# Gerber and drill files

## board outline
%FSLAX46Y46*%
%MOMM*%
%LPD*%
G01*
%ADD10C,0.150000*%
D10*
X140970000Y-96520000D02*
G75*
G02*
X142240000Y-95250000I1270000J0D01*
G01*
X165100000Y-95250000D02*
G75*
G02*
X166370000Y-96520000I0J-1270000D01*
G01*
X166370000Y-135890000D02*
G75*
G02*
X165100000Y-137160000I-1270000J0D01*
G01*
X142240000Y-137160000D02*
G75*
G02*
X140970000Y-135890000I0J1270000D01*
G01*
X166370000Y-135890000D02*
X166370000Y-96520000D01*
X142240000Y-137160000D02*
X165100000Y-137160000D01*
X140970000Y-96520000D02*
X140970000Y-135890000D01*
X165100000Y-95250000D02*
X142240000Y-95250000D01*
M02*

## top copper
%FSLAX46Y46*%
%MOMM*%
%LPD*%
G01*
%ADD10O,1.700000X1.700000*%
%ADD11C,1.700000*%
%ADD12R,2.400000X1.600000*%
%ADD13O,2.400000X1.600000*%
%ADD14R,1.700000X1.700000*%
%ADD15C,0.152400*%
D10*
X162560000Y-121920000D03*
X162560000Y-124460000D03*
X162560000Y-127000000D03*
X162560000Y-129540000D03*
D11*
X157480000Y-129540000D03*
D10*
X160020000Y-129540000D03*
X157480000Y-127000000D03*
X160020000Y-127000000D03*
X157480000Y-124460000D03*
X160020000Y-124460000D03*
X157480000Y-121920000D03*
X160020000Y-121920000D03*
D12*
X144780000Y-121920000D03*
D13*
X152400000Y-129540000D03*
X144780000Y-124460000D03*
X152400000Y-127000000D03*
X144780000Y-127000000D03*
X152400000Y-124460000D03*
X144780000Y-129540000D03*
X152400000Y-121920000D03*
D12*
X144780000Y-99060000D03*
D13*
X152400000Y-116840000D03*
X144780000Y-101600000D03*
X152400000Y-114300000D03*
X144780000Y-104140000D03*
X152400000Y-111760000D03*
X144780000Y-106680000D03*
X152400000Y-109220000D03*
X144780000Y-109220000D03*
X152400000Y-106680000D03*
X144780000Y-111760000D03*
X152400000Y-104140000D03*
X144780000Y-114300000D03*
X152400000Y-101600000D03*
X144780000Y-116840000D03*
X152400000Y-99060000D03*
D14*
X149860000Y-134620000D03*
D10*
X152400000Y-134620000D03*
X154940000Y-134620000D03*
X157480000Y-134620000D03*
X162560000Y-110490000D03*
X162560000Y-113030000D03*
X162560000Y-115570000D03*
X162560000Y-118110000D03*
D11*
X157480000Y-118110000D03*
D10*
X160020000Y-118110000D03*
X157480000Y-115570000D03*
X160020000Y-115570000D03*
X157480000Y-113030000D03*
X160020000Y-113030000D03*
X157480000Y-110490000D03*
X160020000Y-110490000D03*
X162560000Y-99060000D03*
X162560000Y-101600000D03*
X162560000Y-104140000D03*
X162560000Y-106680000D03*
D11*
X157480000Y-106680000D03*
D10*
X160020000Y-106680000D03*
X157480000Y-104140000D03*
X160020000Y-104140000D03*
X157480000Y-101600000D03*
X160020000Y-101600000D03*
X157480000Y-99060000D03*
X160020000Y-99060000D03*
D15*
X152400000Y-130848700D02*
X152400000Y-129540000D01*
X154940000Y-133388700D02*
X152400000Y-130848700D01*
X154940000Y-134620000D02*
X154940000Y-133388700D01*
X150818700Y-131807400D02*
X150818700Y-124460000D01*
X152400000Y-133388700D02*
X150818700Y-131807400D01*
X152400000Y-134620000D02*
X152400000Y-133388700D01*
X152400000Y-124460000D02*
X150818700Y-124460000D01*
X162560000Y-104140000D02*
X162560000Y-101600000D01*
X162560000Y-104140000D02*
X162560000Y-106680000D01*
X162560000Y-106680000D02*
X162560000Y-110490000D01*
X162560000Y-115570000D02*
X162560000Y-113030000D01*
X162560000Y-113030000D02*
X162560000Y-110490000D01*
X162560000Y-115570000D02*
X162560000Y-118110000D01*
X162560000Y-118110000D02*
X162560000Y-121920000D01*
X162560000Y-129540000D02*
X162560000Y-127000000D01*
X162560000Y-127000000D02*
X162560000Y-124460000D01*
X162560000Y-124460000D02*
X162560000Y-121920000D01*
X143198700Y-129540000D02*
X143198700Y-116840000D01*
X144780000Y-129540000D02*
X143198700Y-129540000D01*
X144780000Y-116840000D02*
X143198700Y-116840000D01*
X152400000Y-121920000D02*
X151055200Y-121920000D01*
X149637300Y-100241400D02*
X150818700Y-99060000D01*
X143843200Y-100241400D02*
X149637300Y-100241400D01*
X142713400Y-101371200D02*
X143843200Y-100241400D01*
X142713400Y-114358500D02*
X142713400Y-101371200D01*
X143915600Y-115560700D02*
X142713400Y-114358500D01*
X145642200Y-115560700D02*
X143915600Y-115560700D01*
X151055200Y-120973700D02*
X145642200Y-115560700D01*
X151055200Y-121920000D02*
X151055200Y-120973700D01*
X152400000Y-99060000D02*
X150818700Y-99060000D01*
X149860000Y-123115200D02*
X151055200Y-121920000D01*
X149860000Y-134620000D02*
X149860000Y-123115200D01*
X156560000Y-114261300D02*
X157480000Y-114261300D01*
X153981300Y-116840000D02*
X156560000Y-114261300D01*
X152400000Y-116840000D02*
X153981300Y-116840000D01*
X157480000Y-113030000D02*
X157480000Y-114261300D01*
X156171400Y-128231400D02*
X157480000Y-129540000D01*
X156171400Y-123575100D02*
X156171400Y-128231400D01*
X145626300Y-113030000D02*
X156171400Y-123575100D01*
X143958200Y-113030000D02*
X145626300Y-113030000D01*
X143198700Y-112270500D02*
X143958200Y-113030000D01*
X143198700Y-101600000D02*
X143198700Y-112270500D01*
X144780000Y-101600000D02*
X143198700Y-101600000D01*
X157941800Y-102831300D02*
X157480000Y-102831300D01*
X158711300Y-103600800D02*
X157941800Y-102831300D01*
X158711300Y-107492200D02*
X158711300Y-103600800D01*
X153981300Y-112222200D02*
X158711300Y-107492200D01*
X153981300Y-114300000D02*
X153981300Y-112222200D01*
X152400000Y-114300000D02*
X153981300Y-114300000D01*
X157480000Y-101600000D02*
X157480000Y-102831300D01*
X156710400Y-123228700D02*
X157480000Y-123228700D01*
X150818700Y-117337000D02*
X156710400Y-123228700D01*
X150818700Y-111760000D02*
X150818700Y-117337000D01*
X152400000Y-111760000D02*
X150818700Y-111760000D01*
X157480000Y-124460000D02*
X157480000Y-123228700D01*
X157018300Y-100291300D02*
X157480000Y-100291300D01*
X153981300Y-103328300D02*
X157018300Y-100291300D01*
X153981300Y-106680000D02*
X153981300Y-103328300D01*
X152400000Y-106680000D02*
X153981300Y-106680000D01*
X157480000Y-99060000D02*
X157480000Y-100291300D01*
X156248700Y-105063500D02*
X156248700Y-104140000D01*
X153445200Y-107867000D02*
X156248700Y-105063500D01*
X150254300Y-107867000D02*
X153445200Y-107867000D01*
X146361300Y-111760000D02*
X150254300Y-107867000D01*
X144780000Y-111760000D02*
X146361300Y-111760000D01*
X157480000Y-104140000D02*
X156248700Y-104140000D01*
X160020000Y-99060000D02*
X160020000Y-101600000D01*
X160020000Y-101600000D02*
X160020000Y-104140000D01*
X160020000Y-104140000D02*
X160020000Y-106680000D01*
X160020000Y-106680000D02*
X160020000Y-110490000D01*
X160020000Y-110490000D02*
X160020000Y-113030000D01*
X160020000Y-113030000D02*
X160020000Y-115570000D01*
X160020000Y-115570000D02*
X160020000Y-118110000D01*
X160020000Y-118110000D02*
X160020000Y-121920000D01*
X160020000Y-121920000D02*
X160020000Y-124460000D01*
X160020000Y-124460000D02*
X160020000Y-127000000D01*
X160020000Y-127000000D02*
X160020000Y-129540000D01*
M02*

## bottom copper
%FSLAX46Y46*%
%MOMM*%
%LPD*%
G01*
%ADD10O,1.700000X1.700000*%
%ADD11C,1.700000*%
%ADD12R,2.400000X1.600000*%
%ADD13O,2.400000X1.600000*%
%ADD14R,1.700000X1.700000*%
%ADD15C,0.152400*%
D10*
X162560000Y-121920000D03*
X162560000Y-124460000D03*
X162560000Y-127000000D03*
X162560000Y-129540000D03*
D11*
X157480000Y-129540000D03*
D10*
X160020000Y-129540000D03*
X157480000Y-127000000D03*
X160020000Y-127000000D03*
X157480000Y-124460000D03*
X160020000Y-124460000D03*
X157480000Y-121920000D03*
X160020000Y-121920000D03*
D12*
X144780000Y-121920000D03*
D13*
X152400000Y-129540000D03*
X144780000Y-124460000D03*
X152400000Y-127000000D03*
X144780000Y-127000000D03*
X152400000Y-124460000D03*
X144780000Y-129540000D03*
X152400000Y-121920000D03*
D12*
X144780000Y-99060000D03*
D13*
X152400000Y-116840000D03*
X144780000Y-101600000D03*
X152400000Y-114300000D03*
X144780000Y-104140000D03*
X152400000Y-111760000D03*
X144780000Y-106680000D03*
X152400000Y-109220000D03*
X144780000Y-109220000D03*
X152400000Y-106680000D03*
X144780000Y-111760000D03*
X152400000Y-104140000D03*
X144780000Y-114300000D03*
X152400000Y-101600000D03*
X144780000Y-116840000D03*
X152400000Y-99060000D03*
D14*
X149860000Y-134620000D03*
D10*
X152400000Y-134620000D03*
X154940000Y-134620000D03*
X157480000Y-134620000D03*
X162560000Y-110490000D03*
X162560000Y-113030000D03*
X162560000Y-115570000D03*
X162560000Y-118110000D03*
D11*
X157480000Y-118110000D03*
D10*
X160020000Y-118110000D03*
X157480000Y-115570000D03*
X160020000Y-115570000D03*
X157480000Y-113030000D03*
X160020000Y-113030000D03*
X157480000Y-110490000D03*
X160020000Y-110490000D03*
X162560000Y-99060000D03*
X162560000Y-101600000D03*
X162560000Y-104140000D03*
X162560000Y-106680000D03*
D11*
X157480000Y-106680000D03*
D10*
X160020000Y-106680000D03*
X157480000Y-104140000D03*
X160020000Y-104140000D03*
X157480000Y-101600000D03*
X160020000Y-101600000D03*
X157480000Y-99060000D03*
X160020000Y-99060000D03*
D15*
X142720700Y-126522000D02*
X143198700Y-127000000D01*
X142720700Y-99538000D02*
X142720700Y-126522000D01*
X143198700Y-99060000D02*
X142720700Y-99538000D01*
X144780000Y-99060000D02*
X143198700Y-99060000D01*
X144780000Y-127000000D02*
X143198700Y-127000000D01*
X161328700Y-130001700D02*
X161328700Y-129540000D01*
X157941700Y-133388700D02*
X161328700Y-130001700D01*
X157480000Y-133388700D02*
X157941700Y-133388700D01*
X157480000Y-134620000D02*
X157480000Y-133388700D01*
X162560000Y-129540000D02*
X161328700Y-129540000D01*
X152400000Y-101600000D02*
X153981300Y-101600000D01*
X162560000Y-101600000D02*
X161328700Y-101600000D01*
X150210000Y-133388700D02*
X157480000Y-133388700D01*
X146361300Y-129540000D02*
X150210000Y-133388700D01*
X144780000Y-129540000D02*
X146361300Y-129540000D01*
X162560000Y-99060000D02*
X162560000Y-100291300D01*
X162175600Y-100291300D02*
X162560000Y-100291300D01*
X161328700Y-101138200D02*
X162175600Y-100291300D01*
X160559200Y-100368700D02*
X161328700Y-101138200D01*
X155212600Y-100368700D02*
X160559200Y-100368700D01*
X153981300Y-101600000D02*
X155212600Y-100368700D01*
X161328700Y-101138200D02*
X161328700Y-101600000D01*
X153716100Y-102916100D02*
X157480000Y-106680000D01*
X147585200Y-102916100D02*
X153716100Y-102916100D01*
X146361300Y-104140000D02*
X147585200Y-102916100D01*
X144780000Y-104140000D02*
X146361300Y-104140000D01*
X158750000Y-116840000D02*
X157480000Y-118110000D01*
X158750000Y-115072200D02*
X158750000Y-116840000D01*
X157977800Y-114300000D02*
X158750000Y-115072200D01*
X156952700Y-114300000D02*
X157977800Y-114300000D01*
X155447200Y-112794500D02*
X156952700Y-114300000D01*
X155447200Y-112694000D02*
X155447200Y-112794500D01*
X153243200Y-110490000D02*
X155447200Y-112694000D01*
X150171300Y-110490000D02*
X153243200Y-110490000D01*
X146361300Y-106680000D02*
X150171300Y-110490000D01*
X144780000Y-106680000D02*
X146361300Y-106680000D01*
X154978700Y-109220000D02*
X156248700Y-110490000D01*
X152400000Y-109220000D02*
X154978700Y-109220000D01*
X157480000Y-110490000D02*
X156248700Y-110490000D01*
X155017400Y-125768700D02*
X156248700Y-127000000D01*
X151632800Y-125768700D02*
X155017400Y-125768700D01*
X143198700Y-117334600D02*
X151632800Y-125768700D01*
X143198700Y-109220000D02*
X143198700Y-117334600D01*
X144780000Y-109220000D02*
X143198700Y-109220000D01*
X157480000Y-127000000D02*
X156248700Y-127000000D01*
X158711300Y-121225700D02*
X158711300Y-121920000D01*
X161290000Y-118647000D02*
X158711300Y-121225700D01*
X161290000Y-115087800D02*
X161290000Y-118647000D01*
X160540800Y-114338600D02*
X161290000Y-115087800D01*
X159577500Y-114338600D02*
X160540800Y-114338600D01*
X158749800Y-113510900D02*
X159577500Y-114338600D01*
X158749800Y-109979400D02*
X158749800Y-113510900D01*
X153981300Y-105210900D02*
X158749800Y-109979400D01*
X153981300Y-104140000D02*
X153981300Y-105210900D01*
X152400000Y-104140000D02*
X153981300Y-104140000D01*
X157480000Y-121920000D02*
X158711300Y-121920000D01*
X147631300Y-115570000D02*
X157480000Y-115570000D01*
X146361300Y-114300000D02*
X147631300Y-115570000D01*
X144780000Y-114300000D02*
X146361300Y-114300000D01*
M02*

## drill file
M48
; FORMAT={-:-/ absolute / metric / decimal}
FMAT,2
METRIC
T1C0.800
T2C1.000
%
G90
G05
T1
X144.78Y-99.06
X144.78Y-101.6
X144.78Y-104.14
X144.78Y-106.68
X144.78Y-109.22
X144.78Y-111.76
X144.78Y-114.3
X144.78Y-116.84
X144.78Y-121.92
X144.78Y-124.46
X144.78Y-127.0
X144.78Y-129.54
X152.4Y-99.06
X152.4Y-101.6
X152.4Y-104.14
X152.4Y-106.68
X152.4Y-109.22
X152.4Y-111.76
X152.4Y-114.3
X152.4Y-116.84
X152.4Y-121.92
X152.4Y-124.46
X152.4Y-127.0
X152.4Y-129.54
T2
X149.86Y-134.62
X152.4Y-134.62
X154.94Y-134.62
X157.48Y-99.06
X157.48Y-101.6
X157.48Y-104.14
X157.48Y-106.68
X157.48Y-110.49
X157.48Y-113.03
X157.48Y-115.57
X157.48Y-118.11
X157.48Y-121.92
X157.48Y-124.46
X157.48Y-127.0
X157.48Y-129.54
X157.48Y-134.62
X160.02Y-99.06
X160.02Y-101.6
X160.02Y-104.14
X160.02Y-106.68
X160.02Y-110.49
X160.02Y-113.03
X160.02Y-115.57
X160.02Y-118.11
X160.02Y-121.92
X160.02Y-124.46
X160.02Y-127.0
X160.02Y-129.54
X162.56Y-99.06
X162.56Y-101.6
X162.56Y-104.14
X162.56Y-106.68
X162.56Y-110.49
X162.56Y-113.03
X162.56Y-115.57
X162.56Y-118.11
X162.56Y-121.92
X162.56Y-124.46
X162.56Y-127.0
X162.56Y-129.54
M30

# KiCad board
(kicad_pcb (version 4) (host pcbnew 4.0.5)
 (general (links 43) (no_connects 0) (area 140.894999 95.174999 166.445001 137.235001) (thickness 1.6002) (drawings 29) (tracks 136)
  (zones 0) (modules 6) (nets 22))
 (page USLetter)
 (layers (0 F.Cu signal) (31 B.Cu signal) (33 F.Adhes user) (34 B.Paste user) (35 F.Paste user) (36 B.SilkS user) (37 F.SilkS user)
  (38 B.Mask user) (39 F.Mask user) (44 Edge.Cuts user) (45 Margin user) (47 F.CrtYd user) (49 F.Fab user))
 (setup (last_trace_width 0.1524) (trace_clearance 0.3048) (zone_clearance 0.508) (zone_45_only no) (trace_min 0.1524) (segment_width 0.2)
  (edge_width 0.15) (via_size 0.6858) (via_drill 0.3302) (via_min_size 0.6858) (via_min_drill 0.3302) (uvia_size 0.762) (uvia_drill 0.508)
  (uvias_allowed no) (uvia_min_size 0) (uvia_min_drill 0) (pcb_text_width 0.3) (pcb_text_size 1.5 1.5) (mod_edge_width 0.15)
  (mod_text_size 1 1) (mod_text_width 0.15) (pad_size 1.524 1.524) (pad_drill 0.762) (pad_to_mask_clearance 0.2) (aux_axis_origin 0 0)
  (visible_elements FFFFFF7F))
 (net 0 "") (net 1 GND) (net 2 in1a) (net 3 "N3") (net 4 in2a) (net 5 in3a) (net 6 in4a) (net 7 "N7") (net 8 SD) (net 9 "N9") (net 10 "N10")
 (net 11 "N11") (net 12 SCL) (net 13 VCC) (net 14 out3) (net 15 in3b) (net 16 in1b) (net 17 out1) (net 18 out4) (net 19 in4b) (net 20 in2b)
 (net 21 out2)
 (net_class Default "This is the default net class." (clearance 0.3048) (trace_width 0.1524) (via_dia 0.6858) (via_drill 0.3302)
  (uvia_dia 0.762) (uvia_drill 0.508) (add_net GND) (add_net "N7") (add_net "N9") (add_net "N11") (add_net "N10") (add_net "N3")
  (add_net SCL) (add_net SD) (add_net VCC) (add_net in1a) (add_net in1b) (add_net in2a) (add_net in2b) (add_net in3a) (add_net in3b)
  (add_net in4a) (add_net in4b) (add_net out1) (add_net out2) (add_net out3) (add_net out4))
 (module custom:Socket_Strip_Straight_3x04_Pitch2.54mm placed (layer F.Cu) (at 157.48 129.54 180)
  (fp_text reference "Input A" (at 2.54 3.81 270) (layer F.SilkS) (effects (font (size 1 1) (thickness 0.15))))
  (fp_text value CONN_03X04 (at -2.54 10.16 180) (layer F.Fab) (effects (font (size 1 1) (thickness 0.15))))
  (pad 12 thru_hole oval (at -5.08 7.62 180) (size 1.7 1.7) (drill 1) (layers *.Cu *.Mask) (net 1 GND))
  (pad 11 thru_hole oval (at -5.08 5.08 180) (size 1.7 1.7) (drill 1) (layers *.Cu *.Mask) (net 1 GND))
  (pad 10 thru_hole oval (at -5.08 2.54 180) (size 1.7 1.7) (drill 1) (layers *.Cu *.Mask) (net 1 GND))
  (pad 9 thru_hole oval (at -5.08 0 180) (size 1.7 1.7) (drill 1) (layers *.Cu *.Mask) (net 1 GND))
  (pad 1 thru_hole circle (at 0 0 180) (size 1.7 1.7) (drill 1) (layers *.Cu *.Mask) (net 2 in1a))
  (pad 2 thru_hole oval (at -2.54 0 180) (size 1.7 1.7) (drill 1) (layers *.Cu *.Mask) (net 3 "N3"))
  (pad 3 thru_hole oval (at 0 2.54 180) (size 1.7 1.7) (drill 1) (layers *.Cu *.Mask) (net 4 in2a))
  (pad 4 thru_hole oval (at -2.54 2.54 180) (size 1.7 1.7) (drill 1) (layers *.Cu *.Mask) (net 3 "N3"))
  (pad 5 thru_hole oval (at 0 5.08 180) (size 1.7 1.7) (drill 1) (layers *.Cu *.Mask) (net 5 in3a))
  (pad 6 thru_hole oval (at -2.54 5.08 180) (size 1.7 1.7) (drill 1) (layers *.Cu *.Mask) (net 3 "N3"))
  (pad 7 thru_hole oval (at 0 7.62 180) (size 1.7 1.7) (drill 1) (layers *.Cu *.Mask) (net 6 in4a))
  (pad 8 thru_hole oval (at -2.54 7.62 180) (size 1.7 1.7) (drill 1) (layers *.Cu *.Mask) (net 3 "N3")))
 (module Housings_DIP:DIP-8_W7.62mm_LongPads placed (layer F.Cu) (at 144.78 121.92)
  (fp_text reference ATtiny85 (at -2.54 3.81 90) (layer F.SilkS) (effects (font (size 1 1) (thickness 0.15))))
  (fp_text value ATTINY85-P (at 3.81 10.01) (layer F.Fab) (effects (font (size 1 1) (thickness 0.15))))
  (pad 1 thru_hole rect (at 0 0) (size 2.4 1.6) (drill 0.8) (layers *.Cu *.Mask) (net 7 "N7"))
  (pad 5 thru_hole oval (at 7.62 7.62) (size 2.4 1.6) (drill 0.8) (layers *.Cu *.Mask) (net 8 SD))
  (pad 2 thru_hole oval (at 0 2.54) (size 2.4 1.6) (drill 0.8) (layers *.Cu *.Mask) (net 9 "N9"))
  (pad 6 thru_hole oval (at 7.62 5.08) (size 2.4 1.6) (drill 0.8) (layers *.Cu *.Mask) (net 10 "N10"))
  (pad 3 thru_hole oval (at 0 5.08) (size 2.4 1.6) (drill 0.8) (layers *.Cu *.Mask) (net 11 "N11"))
  (pad 7 thru_hole oval (at 7.62 2.54) (size 2.4 1.6) (drill 0.8) (layers *.Cu *.Mask) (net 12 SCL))
  (pad 4 thru_hole oval (at 0 7.62) (size 2.4 1.6) (drill 0.8) (layers *.Cu *.Mask) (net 1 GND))
  (pad 8 thru_hole oval (at 7.62 0) (size 2.4 1.6) (drill 0.8) (layers *.Cu *.Mask) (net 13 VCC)))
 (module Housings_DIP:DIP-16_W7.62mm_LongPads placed (layer F.Cu) (at 144.78 99.06)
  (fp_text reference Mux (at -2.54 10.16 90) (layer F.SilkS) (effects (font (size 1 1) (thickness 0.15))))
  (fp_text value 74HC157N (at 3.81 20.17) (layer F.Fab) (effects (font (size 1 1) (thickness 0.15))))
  (pad 1 thru_hole rect (at 0 0) (size 2.4 1.6) (drill 0.8) (layers *.Cu *.Mask) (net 11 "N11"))
  (pad 9 thru_hole oval (at 7.62 17.78) (size 2.4 1.6) (drill 0.8) (layers *.Cu *.Mask) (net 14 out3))
  (pad 2 thru_hole oval (at 0 2.54) (size 2.4 1.6) (drill 0.8) (layers *.Cu *.Mask) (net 2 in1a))
  (pad 10 thru_hole oval (at 7.62 15.24) (size 2.4 1.6) (drill 0.8) (layers *.Cu *.Mask) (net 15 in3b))
  (pad 3 thru_hole oval (at 0 5.08) (size 2.4 1.6) (drill 0.8) (layers *.Cu *.Mask) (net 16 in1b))
  (pad 11 thru_hole oval (at 7.62 12.7) (size 2.4 1.6) (drill 0.8) (layers *.Cu *.Mask) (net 5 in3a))
  (pad 4 thru_hole oval (at 0 7.62) (size 2.4 1.6) (drill 0.8) (layers *.Cu *.Mask) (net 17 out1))
  (pad 12 thru_hole oval (at 7.62 10.16) (size 2.4 1.6) (drill 0.8) (layers *.Cu *.Mask) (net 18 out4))
  (pad 5 thru_hole oval (at 0 10.16) (size 2.4 1.6) (drill 0.8) (layers *.Cu *.Mask) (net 4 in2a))
  (pad 13 thru_hole oval (at 7.62 7.62) (size 2.4 1.6) (drill 0.8) (layers *.Cu *.Mask) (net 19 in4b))
  (pad 6 thru_hole oval (at 0 12.7) (size 2.4 1.6) (drill 0.8) (layers *.Cu *.Mask) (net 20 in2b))
  (pad 14 thru_hole oval (at 7.62 5.08) (size 2.4 1.6) (drill 0.8) (layers *.Cu *.Mask) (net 6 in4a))
  (pad 7 thru_hole oval (at 0 15.24) (size 2.4 1.6) (drill 0.8) (layers *.Cu *.Mask) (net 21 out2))
  (pad 15 thru_hole oval (at 7.62 2.54) (size 2.4 1.6) (drill 0.8) (layers *.Cu *.Mask) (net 1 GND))
  (pad 8 thru_hole oval (at 0 17.78) (size 2.4 1.6) (drill 0.8) (layers *.Cu *.Mask) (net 1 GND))
  (pad 16 thru_hole oval (at 7.62 0) (size 2.4 1.6) (drill 0.8) (layers *.Cu *.Mask) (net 13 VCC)))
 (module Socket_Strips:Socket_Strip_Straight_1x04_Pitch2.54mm (layer F.Cu) (at 149.86 134.62 90)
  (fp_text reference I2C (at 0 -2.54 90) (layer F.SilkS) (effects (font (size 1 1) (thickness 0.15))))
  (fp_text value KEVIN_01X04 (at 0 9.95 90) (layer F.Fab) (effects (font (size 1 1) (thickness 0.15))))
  (pad 1 thru_hole rect (at 0 0 90) (size 1.7 1.7) (drill 1) (layers *.Cu *.Mask) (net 13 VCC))
  (pad 2 thru_hole oval (at 0 2.54 90) (size 1.7 1.7) (drill 1) (layers *.Cu *.Mask) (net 12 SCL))
  (pad 3 thru_hole oval (at 0 5.08 90) (size 1.7 1.7) (drill 1) (layers *.Cu *.Mask) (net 8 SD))
  (pad 4 thru_hole oval (at 0 7.62 90) (size 1.7 1.7) (drill 1) (layers *.Cu *.Mask) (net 1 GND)))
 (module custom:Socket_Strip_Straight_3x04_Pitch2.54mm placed (layer F.Cu) (at 157.48 118.11 180)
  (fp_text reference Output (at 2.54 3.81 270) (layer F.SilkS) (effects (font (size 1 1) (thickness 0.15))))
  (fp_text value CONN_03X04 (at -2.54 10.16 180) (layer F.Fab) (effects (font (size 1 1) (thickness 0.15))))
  (pad 12 thru_hole oval (at -5.08 7.62 180) (size 1.7 1.7) (drill 1) (layers *.Cu *.Mask) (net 1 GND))
  (pad 11 thru_hole oval (at -5.08 5.08 180) (size 1.7 1.7) (drill 1) (layers *.Cu *.Mask) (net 1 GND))
  (pad 10 thru_hole oval (at -5.08 2.54 180) (size 1.7 1.7) (drill 1) (layers *.Cu *.Mask) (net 1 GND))
  (pad 9 thru_hole oval (at -5.08 0 180) (size 1.7 1.7) (drill 1) (layers *.Cu *.Mask) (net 1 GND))
  (pad 1 thru_hole circle (at 0 0 180) (size 1.7 1.7) (drill 1) (layers *.Cu *.Mask) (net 17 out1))
  (pad 2 thru_hole oval (at -2.54 0 180) (size 1.7 1.7) (drill 1) (layers *.Cu *.Mask) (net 3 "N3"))
  (pad 3 thru_hole oval (at 0 2.54 180) (size 1.7 1.7) (drill 1) (layers *.Cu *.Mask) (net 21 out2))
  (pad 4 thru_hole oval (at -2.54 2.54 180) (size 1.7 1.7) (drill 1) (layers *.Cu *.Mask) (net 3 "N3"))
  (pad 5 thru_hole oval (at 0 5.08 180) (size 1.7 1.7) (drill 1) (layers *.Cu *.Mask) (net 14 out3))
  (pad 6 thru_hole oval (at -2.54 5.08 180) (size 1.7 1.7) (drill 1) (layers *.Cu *.Mask) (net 3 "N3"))
  (pad 7 thru_hole oval (at 0 7.62 180) (size 1.7 1.7) (drill 1) (layers *.Cu *.Mask) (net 18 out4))
  (pad 8 thru_hole oval (at -2.54 7.62 180) (size 1.7 1.7) (drill 1) (layers *.Cu *.Mask) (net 3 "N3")))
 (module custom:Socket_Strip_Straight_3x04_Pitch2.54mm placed (layer F.Cu) (at 157.48 106.68 180)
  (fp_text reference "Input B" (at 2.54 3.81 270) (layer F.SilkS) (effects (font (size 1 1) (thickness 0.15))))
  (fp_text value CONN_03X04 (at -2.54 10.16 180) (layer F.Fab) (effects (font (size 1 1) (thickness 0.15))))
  (pad 12 thru_hole oval (at -5.08 7.62 180) (size 1.7 1.7) (drill 1) (layers *.Cu *.Mask) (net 1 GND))
  (pad 11 thru_hole oval (at -5.08 5.08 180) (size 1.7 1.7) (drill 1) (layers *.Cu *.Mask) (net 1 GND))
  (pad 10 thru_hole oval (at -5.08 2.54 180) (size 1.7 1.7) (drill 1) (layers *.Cu *.Mask) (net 1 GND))
  (pad 9 thru_hole oval (at -5.08 0 180) (size 1.7 1.7) (drill 1) (layers *.Cu *.Mask) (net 1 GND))
  (pad 1 thru_hole circle (at 0 0 180) (size 1.7 1.7) (drill 1) (layers *.Cu *.Mask) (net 16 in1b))
  (pad 2 thru_hole oval (at -2.54 0 180) (size 1.7 1.7) (drill 1) (layers *.Cu *.Mask) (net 3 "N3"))
  (pad 3 thru_hole oval (at 0 2.54 180) (size 1.7 1.7) (drill 1) (layers *.Cu *.Mask) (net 20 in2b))
  (pad 4 thru_hole oval (at -2.54 2.54 180) (size 1.7 1.7) (drill 1) (layers *.Cu *.Mask) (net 3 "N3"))
  (pad 5 thru_hole oval (at 0 5.08 180) (size 1.7 1.7) (drill 1) (layers *.Cu *.Mask) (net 15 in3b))
  (pad 6 thru_hole oval (at -2.54 5.08 180) (size 1.7 1.7) (drill 1) (layers *.Cu *.Mask) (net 3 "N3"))
  (pad 7 thru_hole oval (at 0 7.62 180) (size 1.7 1.7) (drill 1) (layers *.Cu *.Mask) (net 19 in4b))
  (pad 8 thru_hole oval (at -2.54 7.62 180) (size 1.7 1.7) (drill 1) (layers *.Cu *.Mask) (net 3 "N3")))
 (gr_arc (start 142.24 96.52) (end 140.97 96.52) (angle 90) (layer Edge.Cuts) (width 0.15))
 (gr_arc (start 165.1 96.52) (end 165.1 95.25) (angle 90) (layer Edge.Cuts) (width 0.15))
 (gr_arc (start 165.1 135.89) (end 166.37 135.89) (angle 90) (layer Edge.Cuts) (width 0.15))
 (gr_arc (start 142.24 135.89) (end 142.24 137.16) (angle 90) (layer Edge.Cuts) (width 0.15))
 (gr_line (start 166.37 135.89) (end 166.37 96.52) (angle 90) (layer Edge.Cuts) (width 0.15))
 (gr_line (start 142.24 137.16) (end 165.1 137.16) (angle 90) (layer Edge.Cuts) (width 0.15))
 (gr_line (start 140.97 96.52) (end 140.97 135.89) (angle 90) (layer Edge.Cuts) (width 0.15))
 (gr_line (start 165.1 95.25) (end 142.24 95.25) (angle 90) (layer Edge.Cuts) (width 0.15))
 (segment (start 152.4 130.8487) (end 152.4 129.54) (width 0.1524) (layer F.Cu) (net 8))
 (segment (start 154.94 133.3887) (end 152.4 130.8487) (width 0.1524) (layer F.Cu) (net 8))
 (segment (start 154.94 134.62) (end 154.94 133.3887) (width 0.1524) (layer F.Cu) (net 8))
 (segment (start 142.7207 126.522) (end 143.1987 127) (width 0.1524) (layer B.Cu) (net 11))
 (segment (start 142.7207 99.538) (end 142.7207 126.522) (width 0.1524) (layer B.Cu) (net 11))
 (segment (start 143.1987 99.06) (end 142.7207 99.538) (width 0.1524) (layer B.Cu) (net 11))
 (segment (start 144.78 99.06) (end 143.1987 99.06) (width 0.1524) (layer B.Cu) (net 11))
 (segment (start 144.78 127) (end 143.1987 127) (width 0.1524) (layer B.Cu) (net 11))
 (segment (start 150.8187 131.8074) (end 150.8187 124.46) (width 0.1524) (layer F.Cu) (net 12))
 (segment (start 152.4 133.3887) (end 150.8187 131.8074) (width 0.1524) (layer F.Cu) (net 12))
 (segment (start 152.4 134.62) (end 152.4 133.3887) (width 0.1524) (layer F.Cu) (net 12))
 (segment (start 152.4 124.46) (end 150.8187 124.46) (width 0.1524) (layer F.Cu) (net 12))
 (segment (start 161.3287 130.0017) (end 161.3287 129.54) (width 0.1524) (layer B.Cu) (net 1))
 (segment (start 157.9417 133.3887) (end 161.3287 130.0017) (width 0.1524) (layer B.Cu) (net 1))
 (segment (start 157.48 133.3887) (end 157.9417 133.3887) (width 0.1524) (layer B.Cu) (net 1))
 (segment (start 157.48 134.62) (end 157.48 133.3887) (width 0.1524) (layer B.Cu) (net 1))
 (segment (start 162.56 129.54) (end 161.3287 129.54) (width 0.1524) (layer B.Cu) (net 1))
 (segment (start 152.4 101.6) (end 153.9813 101.6) (width 0.1524) (layer B.Cu) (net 1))
 (segment (start 162.56 101.6) (end 161.3287 101.6) (width 0.1524) (layer B.Cu) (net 1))
 (segment (start 150.21 133.3887) (end 157.48 133.3887) (width 0.1524) (layer B.Cu) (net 1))
 (segment (start 146.3613 129.54) (end 150.21 133.3887) (width 0.1524) (layer B.Cu) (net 1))
 (segment (start 144.78 129.54) (end 146.3613 129.54) (width 0.1524) (layer B.Cu) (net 1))
 (segment (start 162.56 104.14) (end 162.56 101.6) (width 0.1524) (layer F.Cu) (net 1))
 (segment (start 162.56 104.14) (end 162.56 106.68) (width 0.1524) (layer F.Cu) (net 1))
 (segment (start 162.56 106.68) (end 162.56 110.49) (width 0.1524) (layer F.Cu) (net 1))
 (segment (start 162.56 115.57) (end 162.56 113.03) (width 0.1524) (layer F.Cu) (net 1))
 (segment (start 162.56 113.03) (end 162.56 110.49) (width 0.1524) (layer F.Cu) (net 1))
 (segment (start 162.56 115.57) (end 162.56 118.11) (width 0.1524) (layer F.Cu) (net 1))
 (segment (start 162.56 118.11) (end 162.56 121.92) (width 0.1524) (layer F.Cu) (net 1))
 (segment (start 162.56 129.54) (end 162.56 127) (width 0.1524) (layer F.Cu) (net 1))
 (segment (start 162.56 127) (end 162.56 124.46) (width 0.1524) (layer F.Cu) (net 1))
 (segment (start 162.56 124.46) (end 162.56 121.92) (width 0.1524) (layer F.Cu) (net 1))
 (segment (start 162.56 99.06) (end 162.56 100.2913) (width 0.1524) (layer B.Cu) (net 1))
 (segment (start 162.1756 100.2913) (end 162.56 100.2913) (width 0.1524) (layer B.Cu) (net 1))
 (segment (start 161.3287 101.1382) (end 162.1756 100.2913) (width 0.1524) (layer B.Cu) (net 1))
 (segment (start 160.5592 100.3687) (end 161.3287 101.1382) (width 0.1524) (layer B.Cu) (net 1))
 (segment (start 155.2126 100.3687) (end 160.5592 100.3687) (width 0.1524) (layer B.Cu) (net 1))
 (segment (start 153.9813 101.6) (end 155.2126 100.3687) (width 0.1524) (layer B.Cu) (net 1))
 (segment (start 161.3287 101.1382) (end 161.3287 101.6) (width 0.1524) (layer B.Cu) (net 1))
 (segment (start 143.1987 129.54) (end 143.1987 116.84) (width 0.1524) (layer F.Cu) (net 1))
 (segment (start 144.78 129.54) (end 143.1987 129.54) (width 0.1524) (layer F.Cu) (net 1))
 (segment (start 144.78 116.84) (end 143.1987 116.84) (width 0.1524) (layer F.Cu) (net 1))
 (segment (start 152.4 121.92) (end 151.0552 121.92) (width 0.1524) (layer F.Cu) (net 13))
 (segment (start 149.6373 100.2414) (end 150.8187 99.06) (width 0.1524) (layer F.Cu) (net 13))
 (segment (start 143.8432 100.2414) (end 149.6373 100.2414) (width 0.1524) (layer F.Cu) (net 13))
 (segment (start 142.7134 101.3712) (end 143.8432 100.2414) (width 0.1524) (layer F.Cu) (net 13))
 (segment (start 142.7134 114.3585) (end 142.7134 101.3712) (width 0.1524) (layer F.Cu) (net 13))
 (segment (start 143.9156 115.5607) (end 142.7134 114.3585) (width 0.1524) (layer F.Cu) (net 13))
 (segment (start 145.6422 115.5607) (end 143.9156 115.5607) (width 0.1524) (layer F.Cu) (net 13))
 (segment (start 151.0552 120.9737) (end 145.6422 115.5607) (width 0.1524) (layer F.Cu) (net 13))
 (segment (start 151.0552 121.92) (end 151.0552 120.9737) (width 0.1524) (layer F.Cu) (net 13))
 (segment (start 152.4 99.06) (end 150.8187 99.06) (width 0.1524) (layer F.Cu) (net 13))
 (segment (start 149.86 123.1152) (end 151.0552 121.92) (width 0.1524) (layer F.Cu) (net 13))
 (segment (start 149.86 134.62) (end 149.86 123.1152) (width 0.1524) (layer F.Cu) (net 13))
 (segment (start 156.56 114.2613) (end 157.48 114.2613) (width 0.1524) (layer F.Cu) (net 14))
 (segment (start 153.9813 116.84) (end 156.56 114.2613) (width 0.1524) (layer F.Cu) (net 14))
 (segment (start 152.4 116.84) (end 153.9813 116.84) (width 0.1524) (layer F.Cu) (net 14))
 (segment (start 157.48 113.03) (end 157.48 114.2613) (width 0.1524) (layer F.Cu) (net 14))
 (segment (start 156.1714 128.2314) (end 157.48 129.54) (width 0.1524) (layer F.Cu) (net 2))
 (segment (start 156.1714 123.5751) (end 156.1714 128.2314) (width 0.1524) (layer F.Cu) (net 2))
 (segment (start 145.6263 113.03) (end 156.1714 123.5751) (width 0.1524) (layer F.Cu) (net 2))
 (segment (start 143.9582 113.03) (end 145.6263 113.03) (width 0.1524) (layer F.Cu) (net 2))
 (segment (start 143.1987 112.2705) (end 143.9582 113.03) (width 0.1524) (layer F.Cu) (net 2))
 (segment (start 143.1987 101.6) (end 143.1987 112.2705) (width 0.1524) (layer F.Cu) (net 2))
 (segment (start 144.78 101.6) (end 143.1987 101.6) (width 0.1524) (layer F.Cu) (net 2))
 (segment (start 157.9418 102.8313) (end 157.48 102.8313) (width 0.1524) (layer F.Cu) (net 15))
 (segment (start 158.7113 103.6008) (end 157.9418 102.8313) (width 0.1524) (layer F.Cu) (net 15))
 (segment (start 158.7113 107.4922) (end 158.7113 103.6008) (width 0.1524) (layer F.Cu) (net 15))
 (segment (start 153.9813 112.2222) (end 158.7113 107.4922) (width 0.1524) (layer F.Cu) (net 15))
 (segment (start 153.9813 114.3) (end 153.9813 112.2222) (width 0.1524) (layer F.Cu) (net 15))
 (segment (start 152.4 114.3) (end 153.9813 114.3) (width 0.1524) (layer F.Cu) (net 15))
 (segment (start 157.48 101.6) (end 157.48 102.8313) (width 0.1524) (layer F.Cu) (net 15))
 (segment (start 153.7161 102.9161) (end 157.48 106.68) (width 0.1524) (layer B.Cu) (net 16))
 (segment (start 147.5852 102.9161) (end 153.7161 102.9161) (width 0.1524) (layer B.Cu) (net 16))
 (segment (start 146.3613 104.14) (end 147.5852 102.9161) (width 0.1524) (layer B.Cu) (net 16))
 (segment (start 144.78 104.14) (end 146.3613 104.14) (width 0.1524) (layer B.Cu) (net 16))
 (segment (start 156.7104 123.2287) (end 157.48 123.2287) (width 0.1524) (layer F.Cu) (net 5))
 (segment (start 150.8187 117.337) (end 156.7104 123.2287) (width 0.1524) (layer F.Cu) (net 5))
 (segment (start 150.8187 111.76) (end 150.8187 117.337) (width 0.1524) (layer F.Cu) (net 5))
 (segment (start 152.4 111.76) (end 150.8187 111.76) (width 0.1524) (layer F.Cu) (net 5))
 (segment (start 157.48 124.46) (end 157.48 123.2287) (width 0.1524) (layer F.Cu) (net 5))
 (segment (start 158.75 116.84) (end 157.48 118.11) (width 0.1524) (layer B.Cu) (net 17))
 (segment (start 158.75 115.0722) (end 158.75 116.84) (width 0.1524) (layer B.Cu) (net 17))
 (segment (start 157.9778 114.3) (end 158.75 115.0722) (width 0.1524) (layer B.Cu) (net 17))
 (segment (start 156.9527 114.3) (end 157.9778 114.3) (width 0.1524) (layer B.Cu) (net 17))
 (segment (start 155.4472 112.7945) (end 156.9527 114.3) (width 0.1524) (layer B.Cu) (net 17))
 (segment (start 155.4472 112.694) (end 155.4472 112.7945) (width 0.1524) (layer B.Cu) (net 17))
 (segment (start 153.2432 110.49) (end 155.4472 112.694) (width 0.1524) (layer B.Cu) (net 17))
 (segment (start 150.1713 110.49) (end 153.2432 110.49) (width 0.1524) (layer B.Cu) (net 17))
 (segment (start 146.3613 106.68) (end 150.1713 110.49) (width 0.1524) (layer B.Cu) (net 17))
 (segment (start 144.78 106.68) (end 146.3613 106.68) (width 0.1524) (layer B.Cu) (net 17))
 (segment (start 154.9787 109.22) (end 156.2487 110.49) (width 0.1524) (layer B.Cu) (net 18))
 (segment (start 152.4 109.22) (end 154.9787 109.22) (width 0.1524) (layer B.Cu) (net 18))
 (segment (start 157.48 110.49) (end 156.2487 110.49) (width 0.1524) (layer B.Cu) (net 18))
 (segment (start 155.0174 125.7687) (end 156.2487 127) (width 0.1524) (layer B.Cu) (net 4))
 (segment (start 151.6328 125.7687) (end 155.0174 125.7687) (width 0.1524) (layer B.Cu) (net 4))
 (segment (start 143.1987 117.3346) (end 151.6328 125.7687) (width 0.1524) (layer B.Cu) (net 4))
 (segment (start 143.1987 109.22) (end 143.1987 117.3346) (width 0.1524) (layer B.Cu) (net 4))
 (segment (start 144.78 109.22) (end 143.1987 109.22) (width 0.1524) (layer B.Cu) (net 4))
 (segment (start 157.48 127) (end 156.2487 127) (width 0.1524) (layer B.Cu) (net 4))
 (segment (start 157.0183 100.2913) (end 157.48 100.2913) (width 0.1524) (layer F.Cu) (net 19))
 (segment (start 153.9813 103.3283) (end 157.0183 100.2913) (width 0.1524) (layer F.Cu) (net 19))
 (segment (start 153.9813 106.68) (end 153.9813 103.3283) (width 0.1524) (layer F.Cu) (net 19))
 (segment (start 152.4 106.68) (end 153.9813 106.68) (width 0.1524) (layer F.Cu) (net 19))
 (segment (start 157.48 99.06) (end 157.48 100.2913) (width 0.1524) (layer F.Cu) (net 19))
 (segment (start 156.2487 105.0635) (end 156.2487 104.14) (width 0.1524) (layer F.Cu) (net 20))
 (segment (start 153.4452 107.867) (end 156.2487 105.0635) (width 0.1524) (layer F.Cu) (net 20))
 (segment (start 150.2543 107.867) (end 153.4452 107.867) (width 0.1524) (layer F.Cu) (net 20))
 (segment (start 146.3613 111.76) (end 150.2543 107.867) (width 0.1524) (layer F.Cu) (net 20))
 (segment (start 144.78 111.76) (end 146.3613 111.76) (width 0.1524) (layer F.Cu) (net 20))
 (segment (start 157.48 104.14) (end 156.2487 104.14) (width 0.1524) (layer F.Cu) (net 20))
 (segment (start 158.7113 121.2257) (end 158.7113 121.92) (width 0.1524) (layer B.Cu) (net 6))
 (segment (start 161.29 118.647) (end 158.7113 121.2257) (width 0.1524) (layer B.Cu) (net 6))
 (segment (start 161.29 115.0878) (end 161.29 118.647) (width 0.1524) (layer B.Cu) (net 6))
 (segment (start 160.5408 114.3386) (end 161.29 115.0878) (width 0.1524) (layer B.Cu) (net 6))
 (segment (start 159.5775 114.3386) (end 160.5408 114.3386) (width 0.1524) (layer B.Cu) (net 6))
 (segment (start 158.7498 113.5109) (end 159.5775 114.3386) (width 0.1524) (layer B.Cu) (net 6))
 (segment (start 158.7498 109.9794) (end 158.7498 113.5109) (width 0.1524) (layer B.Cu) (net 6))
 (segment (start 153.9813 105.2109) (end 158.7498 109.9794) (width 0.1524) (layer B.Cu) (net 6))
 (segment (start 153.9813 104.14) (end 153.9813 105.2109) (width 0.1524) (layer B.Cu) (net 6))
 (segment (start 152.4 104.14) (end 153.9813 104.14) (width 0.1524) (layer B.Cu) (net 6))
 (segment (start 157.48 121.92) (end 158.7113 121.92) (width 0.1524) (layer B.Cu) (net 6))
 (segment (start 147.6313 115.57) (end 157.48 115.57) (width 0.1524) (layer B.Cu) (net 21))
 (segment (start 146.3613 114.3) (end 147.6313 115.57) (width 0.1524) (layer B.Cu) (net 21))
 (segment (start 144.78 114.3) (end 146.3613 114.3) (width 0.1524) (layer B.Cu) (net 21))
 (segment (start 160.02 99.06) (end 160.02 101.6) (width 0.1524) (layer F.Cu) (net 3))
 (segment (start 160.02 101.6) (end 160.02 104.14) (width 0.1524) (layer F.Cu) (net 3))
 (segment (start 160.02 104.14) (end 160.02 106.68) (width 0.1524) (layer F.Cu) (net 3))
 (segment (start 160.02 106.68) (end 160.02 110.49) (width 0.1524) (layer F.Cu) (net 3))
 (segment (start 160.02 110.49) (end 160.02 113.03) (width 0.1524) (layer F.Cu) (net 3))
 (segment (start 160.02 113.03) (end 160.02 115.57) (width 0.1524) (layer F.Cu) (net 3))
 (segment (start 160.02 115.57) (end 160.02 118.11) (width 0.1524) (layer F.Cu) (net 3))
 (segment (start 160.02 118.11) (end 160.02 121.92) (width 0.1524) (layer F.Cu) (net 3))
 (segment (start 160.02 121.92) (end 160.02 124.46) (width 0.1524) (layer F.Cu) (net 3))
 (segment (start 160.02 124.46) (end 160.02 127) (width 0.1524) (layer F.Cu) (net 3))
 (segment (start 160.02 127) (end 160.02 129.54) (width 0.1524) (layer F.Cu) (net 3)))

